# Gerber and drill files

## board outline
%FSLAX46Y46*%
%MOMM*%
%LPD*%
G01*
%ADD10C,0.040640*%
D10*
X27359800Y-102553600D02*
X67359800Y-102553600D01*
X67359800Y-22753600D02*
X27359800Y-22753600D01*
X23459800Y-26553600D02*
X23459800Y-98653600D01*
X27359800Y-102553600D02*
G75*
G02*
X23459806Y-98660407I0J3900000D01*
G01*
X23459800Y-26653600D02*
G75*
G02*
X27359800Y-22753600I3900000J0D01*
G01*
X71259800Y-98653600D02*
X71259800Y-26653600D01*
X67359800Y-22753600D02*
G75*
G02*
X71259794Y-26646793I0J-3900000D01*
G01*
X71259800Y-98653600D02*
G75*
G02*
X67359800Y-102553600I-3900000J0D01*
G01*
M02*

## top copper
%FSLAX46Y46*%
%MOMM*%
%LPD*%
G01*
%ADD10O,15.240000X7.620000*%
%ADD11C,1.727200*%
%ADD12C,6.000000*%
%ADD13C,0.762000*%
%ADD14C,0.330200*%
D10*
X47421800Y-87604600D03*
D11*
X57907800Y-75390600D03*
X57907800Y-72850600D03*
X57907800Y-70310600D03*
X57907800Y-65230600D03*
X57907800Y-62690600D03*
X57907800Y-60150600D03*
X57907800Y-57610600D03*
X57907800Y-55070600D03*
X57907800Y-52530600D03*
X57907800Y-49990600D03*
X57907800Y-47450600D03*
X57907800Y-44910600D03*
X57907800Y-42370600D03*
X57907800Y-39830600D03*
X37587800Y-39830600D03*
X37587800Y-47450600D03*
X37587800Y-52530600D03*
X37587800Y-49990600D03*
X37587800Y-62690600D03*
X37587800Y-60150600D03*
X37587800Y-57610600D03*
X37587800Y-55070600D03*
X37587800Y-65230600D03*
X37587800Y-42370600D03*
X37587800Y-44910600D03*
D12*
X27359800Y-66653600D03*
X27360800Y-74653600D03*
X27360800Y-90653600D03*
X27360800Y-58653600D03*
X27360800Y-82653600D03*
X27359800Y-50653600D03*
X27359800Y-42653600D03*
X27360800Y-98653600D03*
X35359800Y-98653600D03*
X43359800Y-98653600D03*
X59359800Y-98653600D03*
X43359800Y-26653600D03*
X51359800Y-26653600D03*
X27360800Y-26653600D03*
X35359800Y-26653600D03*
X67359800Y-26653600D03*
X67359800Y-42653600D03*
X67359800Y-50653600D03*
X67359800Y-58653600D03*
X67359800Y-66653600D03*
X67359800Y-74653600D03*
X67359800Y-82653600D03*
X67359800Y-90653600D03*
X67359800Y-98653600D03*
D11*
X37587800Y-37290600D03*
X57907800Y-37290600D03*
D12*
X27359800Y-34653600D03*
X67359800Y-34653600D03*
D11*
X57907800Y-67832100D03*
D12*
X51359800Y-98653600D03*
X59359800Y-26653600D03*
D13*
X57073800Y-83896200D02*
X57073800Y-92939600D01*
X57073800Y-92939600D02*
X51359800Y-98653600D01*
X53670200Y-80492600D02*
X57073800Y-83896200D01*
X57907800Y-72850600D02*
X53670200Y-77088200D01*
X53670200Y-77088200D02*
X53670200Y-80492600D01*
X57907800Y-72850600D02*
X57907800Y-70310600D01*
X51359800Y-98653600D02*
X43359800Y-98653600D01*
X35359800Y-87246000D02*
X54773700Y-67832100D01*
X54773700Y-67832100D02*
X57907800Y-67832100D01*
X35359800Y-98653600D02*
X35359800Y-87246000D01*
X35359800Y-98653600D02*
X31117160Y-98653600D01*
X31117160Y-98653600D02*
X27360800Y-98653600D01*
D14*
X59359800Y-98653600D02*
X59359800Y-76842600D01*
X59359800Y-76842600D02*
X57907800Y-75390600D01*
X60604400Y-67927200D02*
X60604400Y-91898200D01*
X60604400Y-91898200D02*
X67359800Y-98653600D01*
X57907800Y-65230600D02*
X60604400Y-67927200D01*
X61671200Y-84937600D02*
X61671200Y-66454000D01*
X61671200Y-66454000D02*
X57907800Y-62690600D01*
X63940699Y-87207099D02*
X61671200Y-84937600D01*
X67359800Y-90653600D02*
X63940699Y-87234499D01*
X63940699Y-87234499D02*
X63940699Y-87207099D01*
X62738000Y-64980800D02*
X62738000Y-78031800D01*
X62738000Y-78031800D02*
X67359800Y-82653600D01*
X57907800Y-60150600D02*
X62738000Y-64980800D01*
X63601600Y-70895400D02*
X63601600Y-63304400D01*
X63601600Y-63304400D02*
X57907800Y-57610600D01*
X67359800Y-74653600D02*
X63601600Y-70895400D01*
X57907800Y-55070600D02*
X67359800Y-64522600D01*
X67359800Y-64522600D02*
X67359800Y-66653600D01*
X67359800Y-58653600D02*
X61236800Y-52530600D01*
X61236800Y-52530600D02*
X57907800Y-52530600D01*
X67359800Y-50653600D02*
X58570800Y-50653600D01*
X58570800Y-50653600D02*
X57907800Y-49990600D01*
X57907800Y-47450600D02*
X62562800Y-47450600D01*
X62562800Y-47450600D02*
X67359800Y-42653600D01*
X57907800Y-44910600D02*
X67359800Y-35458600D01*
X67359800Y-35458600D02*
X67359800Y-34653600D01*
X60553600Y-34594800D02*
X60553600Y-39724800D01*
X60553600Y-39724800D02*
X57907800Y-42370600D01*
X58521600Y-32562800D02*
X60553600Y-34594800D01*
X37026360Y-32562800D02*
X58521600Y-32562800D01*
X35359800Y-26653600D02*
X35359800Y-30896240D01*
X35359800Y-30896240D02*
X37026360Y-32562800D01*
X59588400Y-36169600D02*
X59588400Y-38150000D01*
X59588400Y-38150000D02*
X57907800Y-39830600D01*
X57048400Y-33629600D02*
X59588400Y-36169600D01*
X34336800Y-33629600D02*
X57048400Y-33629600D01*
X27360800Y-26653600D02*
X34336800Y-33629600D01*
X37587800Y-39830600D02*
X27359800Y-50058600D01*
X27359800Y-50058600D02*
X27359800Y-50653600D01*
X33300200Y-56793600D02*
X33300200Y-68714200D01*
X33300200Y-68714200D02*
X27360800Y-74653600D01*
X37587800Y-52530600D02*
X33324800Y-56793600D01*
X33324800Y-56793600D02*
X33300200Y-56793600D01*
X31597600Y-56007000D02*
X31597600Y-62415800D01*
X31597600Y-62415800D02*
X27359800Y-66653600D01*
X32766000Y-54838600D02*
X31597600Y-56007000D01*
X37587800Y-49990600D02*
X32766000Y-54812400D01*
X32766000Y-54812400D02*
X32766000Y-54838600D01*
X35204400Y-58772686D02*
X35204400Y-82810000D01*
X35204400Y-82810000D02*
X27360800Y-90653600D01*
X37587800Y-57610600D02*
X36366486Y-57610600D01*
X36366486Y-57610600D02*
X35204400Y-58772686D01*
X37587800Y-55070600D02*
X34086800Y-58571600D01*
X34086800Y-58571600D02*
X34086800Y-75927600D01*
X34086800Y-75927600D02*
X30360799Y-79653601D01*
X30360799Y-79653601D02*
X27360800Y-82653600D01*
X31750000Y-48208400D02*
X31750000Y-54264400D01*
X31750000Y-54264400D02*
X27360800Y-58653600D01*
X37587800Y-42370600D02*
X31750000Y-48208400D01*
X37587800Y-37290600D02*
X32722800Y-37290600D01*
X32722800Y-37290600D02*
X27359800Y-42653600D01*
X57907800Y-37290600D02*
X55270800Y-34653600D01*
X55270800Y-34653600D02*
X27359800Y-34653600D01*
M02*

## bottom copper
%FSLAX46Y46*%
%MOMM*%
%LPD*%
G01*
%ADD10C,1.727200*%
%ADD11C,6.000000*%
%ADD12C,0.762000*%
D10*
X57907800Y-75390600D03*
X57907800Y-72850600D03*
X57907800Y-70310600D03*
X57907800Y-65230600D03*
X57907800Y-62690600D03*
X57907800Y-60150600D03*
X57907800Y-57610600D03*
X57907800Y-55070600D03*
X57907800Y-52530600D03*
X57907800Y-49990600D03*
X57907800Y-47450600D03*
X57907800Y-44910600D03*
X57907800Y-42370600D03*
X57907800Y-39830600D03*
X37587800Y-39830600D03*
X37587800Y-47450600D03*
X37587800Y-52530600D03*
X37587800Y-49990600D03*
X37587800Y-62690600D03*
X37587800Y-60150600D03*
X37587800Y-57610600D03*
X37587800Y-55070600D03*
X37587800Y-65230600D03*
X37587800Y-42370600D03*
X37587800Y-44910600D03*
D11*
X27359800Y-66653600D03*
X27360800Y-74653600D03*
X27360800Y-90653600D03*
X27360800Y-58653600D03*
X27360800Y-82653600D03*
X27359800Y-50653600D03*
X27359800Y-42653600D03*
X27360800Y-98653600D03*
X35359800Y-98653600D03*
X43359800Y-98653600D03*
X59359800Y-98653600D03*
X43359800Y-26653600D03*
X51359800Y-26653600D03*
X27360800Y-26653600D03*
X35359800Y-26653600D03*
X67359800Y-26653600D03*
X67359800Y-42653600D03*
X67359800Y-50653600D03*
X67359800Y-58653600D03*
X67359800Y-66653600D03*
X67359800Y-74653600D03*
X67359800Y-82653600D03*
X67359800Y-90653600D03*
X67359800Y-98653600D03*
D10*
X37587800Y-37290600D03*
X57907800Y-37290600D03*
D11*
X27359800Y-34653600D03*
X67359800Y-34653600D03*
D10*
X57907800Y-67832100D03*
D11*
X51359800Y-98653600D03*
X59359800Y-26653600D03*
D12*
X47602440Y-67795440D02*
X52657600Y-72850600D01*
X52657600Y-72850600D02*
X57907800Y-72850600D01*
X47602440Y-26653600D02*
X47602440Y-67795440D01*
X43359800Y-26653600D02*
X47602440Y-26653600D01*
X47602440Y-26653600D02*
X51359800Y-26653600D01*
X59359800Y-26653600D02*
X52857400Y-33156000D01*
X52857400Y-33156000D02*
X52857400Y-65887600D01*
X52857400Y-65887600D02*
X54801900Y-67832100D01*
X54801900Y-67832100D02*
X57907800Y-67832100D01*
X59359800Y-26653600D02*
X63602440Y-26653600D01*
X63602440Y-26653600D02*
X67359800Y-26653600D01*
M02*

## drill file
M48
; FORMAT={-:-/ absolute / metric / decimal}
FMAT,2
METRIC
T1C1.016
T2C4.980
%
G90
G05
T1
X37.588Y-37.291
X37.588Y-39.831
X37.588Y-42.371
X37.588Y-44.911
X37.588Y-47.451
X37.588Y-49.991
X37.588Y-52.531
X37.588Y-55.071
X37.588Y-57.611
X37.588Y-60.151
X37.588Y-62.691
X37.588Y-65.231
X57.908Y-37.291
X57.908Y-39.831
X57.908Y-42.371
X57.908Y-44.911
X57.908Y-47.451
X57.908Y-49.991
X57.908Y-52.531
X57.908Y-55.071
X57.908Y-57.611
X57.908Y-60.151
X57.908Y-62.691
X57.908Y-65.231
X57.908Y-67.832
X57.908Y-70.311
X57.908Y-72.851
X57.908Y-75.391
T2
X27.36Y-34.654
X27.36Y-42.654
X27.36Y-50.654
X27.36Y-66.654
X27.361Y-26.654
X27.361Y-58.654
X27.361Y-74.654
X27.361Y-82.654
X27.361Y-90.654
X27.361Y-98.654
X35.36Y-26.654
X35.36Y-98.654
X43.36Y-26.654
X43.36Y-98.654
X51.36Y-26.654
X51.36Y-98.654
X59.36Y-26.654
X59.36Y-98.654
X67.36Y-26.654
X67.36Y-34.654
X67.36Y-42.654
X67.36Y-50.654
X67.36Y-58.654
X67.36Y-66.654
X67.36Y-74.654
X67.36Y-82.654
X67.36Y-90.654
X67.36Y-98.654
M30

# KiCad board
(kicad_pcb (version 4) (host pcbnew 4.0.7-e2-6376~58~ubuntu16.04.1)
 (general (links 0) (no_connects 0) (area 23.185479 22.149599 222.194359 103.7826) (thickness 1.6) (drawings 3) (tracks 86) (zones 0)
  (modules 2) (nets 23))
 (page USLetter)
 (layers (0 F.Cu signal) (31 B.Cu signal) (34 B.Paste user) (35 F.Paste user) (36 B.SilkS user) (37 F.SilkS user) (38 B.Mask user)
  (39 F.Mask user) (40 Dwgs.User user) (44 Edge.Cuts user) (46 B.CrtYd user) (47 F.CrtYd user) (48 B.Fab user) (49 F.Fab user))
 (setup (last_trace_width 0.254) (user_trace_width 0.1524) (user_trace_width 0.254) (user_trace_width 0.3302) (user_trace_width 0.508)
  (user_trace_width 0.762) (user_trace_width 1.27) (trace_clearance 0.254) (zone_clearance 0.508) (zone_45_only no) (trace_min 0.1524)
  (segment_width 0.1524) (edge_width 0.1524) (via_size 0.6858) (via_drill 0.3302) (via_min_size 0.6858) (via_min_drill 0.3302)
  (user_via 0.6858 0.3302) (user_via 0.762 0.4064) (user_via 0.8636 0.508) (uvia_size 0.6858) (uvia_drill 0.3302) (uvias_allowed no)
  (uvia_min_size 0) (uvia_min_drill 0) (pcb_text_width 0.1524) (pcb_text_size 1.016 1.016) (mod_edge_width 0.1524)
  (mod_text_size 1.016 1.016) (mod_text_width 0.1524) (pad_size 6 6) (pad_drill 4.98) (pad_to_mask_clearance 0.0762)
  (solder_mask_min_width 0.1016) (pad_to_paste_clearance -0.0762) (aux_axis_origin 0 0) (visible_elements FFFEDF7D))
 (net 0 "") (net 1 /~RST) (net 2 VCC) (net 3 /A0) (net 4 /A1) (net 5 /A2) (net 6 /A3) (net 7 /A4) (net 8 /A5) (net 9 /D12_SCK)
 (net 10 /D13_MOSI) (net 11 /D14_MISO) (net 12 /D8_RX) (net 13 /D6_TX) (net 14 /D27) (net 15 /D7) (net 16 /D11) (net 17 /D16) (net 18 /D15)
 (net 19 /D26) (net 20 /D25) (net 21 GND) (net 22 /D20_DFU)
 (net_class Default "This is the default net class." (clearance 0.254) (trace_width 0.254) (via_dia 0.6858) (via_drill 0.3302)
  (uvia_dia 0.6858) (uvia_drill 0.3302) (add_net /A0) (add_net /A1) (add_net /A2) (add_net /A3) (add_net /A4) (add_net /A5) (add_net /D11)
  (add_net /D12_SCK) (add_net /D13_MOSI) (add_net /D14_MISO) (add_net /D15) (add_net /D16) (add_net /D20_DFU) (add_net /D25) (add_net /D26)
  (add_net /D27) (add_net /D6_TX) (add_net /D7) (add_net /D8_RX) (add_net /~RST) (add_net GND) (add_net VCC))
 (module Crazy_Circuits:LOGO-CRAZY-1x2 (layer F.Cu) (at 47.4218 91.5416)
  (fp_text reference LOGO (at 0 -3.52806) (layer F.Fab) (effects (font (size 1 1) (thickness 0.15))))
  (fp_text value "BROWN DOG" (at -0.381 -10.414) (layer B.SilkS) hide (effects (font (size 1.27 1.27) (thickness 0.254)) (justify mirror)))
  (pad BG smd oval (at 0 -3.937) (size 15.24 7.62) (layers F.Cu)))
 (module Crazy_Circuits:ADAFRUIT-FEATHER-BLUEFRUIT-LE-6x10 (layer F.Cu) (at 27.3598 58.6536)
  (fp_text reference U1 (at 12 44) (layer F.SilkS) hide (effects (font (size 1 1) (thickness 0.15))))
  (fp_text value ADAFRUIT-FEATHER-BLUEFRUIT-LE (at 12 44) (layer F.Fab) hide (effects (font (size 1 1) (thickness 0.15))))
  (fp_line (start 0 43.9) (end 40 43.9) (layer Edge.Cuts) (width 0.04064))
  (fp_line (start 40 -35.9) (end 0 -35.9) (layer Edge.Cuts) (width 0.04064))
  (fp_line (start -3.9 -32.1) (end -3.9 40) (layer Edge.Cuts) (width 0.04064))
  (fp_arc (start 0 40) (end 0 43.9) (angle 89.9) (layer Edge.Cuts) (width 0.04064))
  (fp_arc (start 0 -32) (end -3.9 -32) (angle 90) (layer Edge.Cuts) (width 0.04064))
  (fp_line (start 43.9 40) (end 43.9 -32) (layer Edge.Cuts) (width 0.04064))
  (fp_arc (start 40 -32) (end 40 -35.9) (angle 89.9) (layer Edge.Cuts) (width 0.04064))
  (fp_arc (start 40 40) (end 43.9 40) (angle 90) (layer Edge.Cuts) (width 0.04064))
  (pad 35 thru_hole circle (at 30.548 16.737 180) (size 1.7272 1.7272) (drill 1.016) (layers *.Cu *.Mask F.SilkS) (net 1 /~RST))
  (pad 3V thru_hole circle (at 30.548 14.197 180) (size 1.7272 1.7272) (drill 1.016) (layers *.Cu *.Mask F.SilkS) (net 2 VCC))
  (pad 3V thru_hole circle (at 30.548 11.657 180) (size 1.7272 1.7272) (drill 1.016) (layers *.Cu *.Mask F.SilkS) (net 2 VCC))
  (pad 15 thru_hole circle (at 30.548 6.577 180) (size 1.7272 1.7272) (drill 1.016) (layers *.Cu *.Mask F.SilkS) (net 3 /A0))
  (pad 16 thru_hole circle (at 30.548 4.037 180) (size 1.7272 1.7272) (drill 1.016) (layers *.Cu *.Mask F.SilkS) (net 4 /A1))
  (pad 17 thru_hole circle (at 30.548 1.497 180) (size 1.7272 1.7272) (drill 1.016) (layers *.Cu *.Mask F.SilkS) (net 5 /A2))
  (pad 18 thru_hole circle (at 30.548 -1.043 180) (size 1.7272 1.7272) (drill 1.016) (layers *.Cu *.Mask F.SilkS) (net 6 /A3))
  (pad 5 thru_hole circle (at 30.548 -3.583 180) (size 1.7272 1.7272) (drill 1.016) (layers *.Cu *.Mask F.SilkS) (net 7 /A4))
  (pad 6 thru_hole circle (at 30.548 -6.123 180) (size 1.7272 1.7272) (drill 1.016) (layers *.Cu *.Mask F.SilkS) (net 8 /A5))
  (pad 26 thru_hole circle (at 30.548 -8.663 180) (size 1.7272 1.7272) (drill 1.016) (layers *.Cu *.Mask F.SilkS) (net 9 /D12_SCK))
  (pad 27 thru_hole circle (at 30.548 -11.203 180) (size 1.7272 1.7272) (drill 1.016) (layers *.Cu *.Mask F.SilkS) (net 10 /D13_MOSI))
  (pad 28 thru_hole circle (at 30.548 -13.743 180) (size 1.7272 1.7272) (drill 1.016) (layers *.Cu *.Mask F.SilkS) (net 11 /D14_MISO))
  (pad 21 thru_hole circle (at 30.548 -16.283 180) (size 1.7272 1.7272) (drill 1.016) (layers *.Cu *.Mask F.SilkS) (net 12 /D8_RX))
  (pad 19 thru_hole circle (at 30.548 -18.823 180) (size 1.7272 1.7272) (drill 1.016) (layers *.Cu *.Mask F.SilkS) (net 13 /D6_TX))
  (pad 3 thru_hole circle (at 10.228 -18.823 180) (size 1.7272 1.7272) (drill 1.016) (layers *.Cu *.Mask F.SilkS) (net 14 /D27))
  (pad 31 thru_hole circle (at 10.228 -11.203 180) (size 1.7272 1.7272) (drill 1.016) (layers *.Cu *.Mask F.SilkS))
  (pad 20 thru_hole circle (at 10.228 -6.123 180) (size 1.7272 1.7272) (drill 1.016) (layers *.Cu *.Mask F.SilkS) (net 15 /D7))
  (pad 25 thru_hole circle (at 10.228 -8.663 180) (size 1.7272 1.7272) (drill 1.016) (layers *.Cu *.Mask F.SilkS) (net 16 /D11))
  (pad EN thru_hole circle (at 10.228 4.037 180) (size 1.7272 1.7272) (drill 1.016) (layers *.Cu *.Mask F.SilkS))
  (pad USB thru_hole circle (at 10.228 1.497 180) (size 1.7272 1.7272) (drill 1.016) (layers *.Cu *.Mask F.SilkS))
  (pad 30 thru_hole circle (at 10.228 -1.043 180) (size 1.7272 1.7272) (drill 1.016) (layers *.Cu *.Mask F.SilkS) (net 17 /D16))
  (pad 29 thru_hole circle (at 10.228 -3.583 180) (size 1.7272 1.7272) (drill 1.016) (layers *.Cu *.Mask F.SilkS) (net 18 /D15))
  (pad VBAT thru_hole circle (at 10.228 6.577 180) (size 1.7272 1.7272) (drill 1.016) (layers *.Cu *.Mask F.SilkS))
  (pad 4 thru_hole circle (at 10.228 -16.283 180) (size 1.7272 1.7272) (drill 1.016) (layers *.Cu *.Mask F.SilkS) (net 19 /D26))
  (pad 7 thru_hole circle (at 10.228 -13.743 180) (size 1.7272 1.7272) (drill 1.016) (layers *.Cu *.Mask F.SilkS))
  (pad 25 thru_hole circle (at 0 8 90) (size 6 6) (drill 4.98) (layers *.Cu *.Mask) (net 16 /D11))
  (pad 20 thru_hole circle (at 0.001 16 90) (size 6 6) (drill 4.98) (layers *.Cu *.Mask) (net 15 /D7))
  (pad 30 thru_hole circle (at 0.001 32 90) (size 6 6) (drill 4.98) (layers *.Cu *.Mask) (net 17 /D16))
  (pad 4 thru_hole circle (at 0.001 0 90) (size 6 6) (drill 4.98) (layers *.Cu *.Mask) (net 19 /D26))
  (pad 29 thru_hole circle (at 0.001 24 90) (size 6 6) (drill 4.98) (layers *.Cu *.Mask) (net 18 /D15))
  (pad 3 thru_hole circle (at 0 -8 90) (size 6 6) (drill 4.98) (layers *.Cu *.Mask) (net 14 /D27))
  (pad 2 thru_hole circle (at 0 -16 90) (size 6 6) (drill 4.98) (layers *.Cu *.Mask) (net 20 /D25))
  (pad GND thru_hole circle (at 0.001 40 90) (size 6 6) (drill 4.98) (layers *.Cu *.Mask) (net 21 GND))
  (pad GND thru_hole circle (at 8 40 90) (size 6 6) (drill 4.98) (layers *.Cu *.Mask) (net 21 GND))
  (pad 3V thru_hole circle (at 16 40 90) (size 6 6) (drill 4.98) (layers *.Cu *.Mask) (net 2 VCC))
  (pad 35 thru_hole circle (at 32 40 90) (size 6 6) (drill 4.98) (layers *.Cu *.Mask) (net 1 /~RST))
  (pad 3V thru_hole circle (at 16 -32 90) (size 6 6) (drill 4.98) (layers *.Cu *.Mask) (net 2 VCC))
  (pad 3V thru_hole circle (at 24 -32 90) (size 6 6) (drill 4.98) (layers *.Cu *.Mask) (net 2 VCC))
  (pad 19 thru_hole circle (at 0.001 -32 90) (size 6 6) (drill 4.98) (layers *.Cu *.Mask) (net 13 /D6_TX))
  (pad 21 thru_hole circle (at 8 -32 90) (size 6 6) (drill 4.98) (layers *.Cu *.Mask) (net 12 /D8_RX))
  (pad GND thru_hole circle (at 40 -32 90) (size 6 6) (drill 4.98) (layers *.Cu *.Mask) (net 21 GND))
  (pad 27 thru_hole circle (at 40 -16 90) (size 6 6) (drill 4.98) (layers *.Cu *.Mask) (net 10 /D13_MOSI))
  (pad 26 thru_hole circle (at 40 -8 90) (size 6 6) (drill 4.98) (layers *.Cu *.Mask) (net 9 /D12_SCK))
  (pad 6 thru_hole circle (at 40 0 90) (size 6 6) (drill 4.98) (layers *.Cu *.Mask) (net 8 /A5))
  (pad 5 thru_hole circle (at 40 8 90) (size 6 6) (drill 4.98) (layers *.Cu *.Mask) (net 7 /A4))
  (pad 18 thru_hole circle (at 40 16 90) (size 6 6) (drill 4.98) (layers *.Cu *.Mask) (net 6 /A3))
  (pad 17 thru_hole circle (at 40 24 90) (size 6 6) (drill 4.98) (layers *.Cu *.Mask) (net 5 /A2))
  (pad 16 thru_hole circle (at 40 32 90) (size 6 6) (drill 4.98) (layers *.Cu *.Mask) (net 4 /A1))
  (pad 15 thru_hole circle (at 40 40 90) (size 6 6) (drill 4.98) (layers *.Cu *.Mask) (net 3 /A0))
  (pad 2 thru_hole circle (at 10.228 -21.363 180) (size 1.7272 1.7272) (drill 1.016) (layers *.Cu *.Mask F.SilkS) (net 20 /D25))
  (pad 34 thru_hole circle (at 30.548 -21.363 180) (size 1.7272 1.7272) (drill 1.016) (layers *.Cu *.Mask F.SilkS) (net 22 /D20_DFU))
  (pad 34 thru_hole circle (at 0 -24 90) (size 6 6) (drill 4.98) (layers *.Cu *.Mask) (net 22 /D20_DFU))
  (pad 28 thru_hole circle (at 40 -24 90) (size 6 6) (drill 4.98) (layers *.Cu *.Mask) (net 11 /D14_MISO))
  (pad GND thru_hole circle (at 30.548 9.1785 180) (size 1.7272 1.7272) (drill 1.016) (layers *.Cu *.Mask F.SilkS) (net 21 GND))
  (pad 3V thru_hole circle (at 24 40 90) (size 6 6) (drill 4.98) (layers *.Cu *.Mask) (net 2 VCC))
  (pad GND thru_hole circle (at 32 -32 90) (size 6 6) (drill 4.98) (layers *.Cu *.Mask) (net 21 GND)))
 (segment (start 47.60244 67.79544) (end 52.6576 72.8506) (width 0.762) (layer B.Cu) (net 2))
 (segment (start 52.6576 72.8506) (end 57.9078 72.8506) (width 0.762) (layer B.Cu) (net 2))
 (segment (start 47.60244 26.6536) (end 47.60244 67.79544) (width 0.762) (layer B.Cu) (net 2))
 (segment (start 57.0738 83.8962) (end 57.0738 92.9396) (width 0.762) (layer F.Cu) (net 2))
 (segment (start 57.0738 92.9396) (end 51.3598 98.6536) (width 0.762) (layer F.Cu) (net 2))
 (segment (start 53.6702 80.4926) (end 57.0738 83.8962) (width 0.762) (layer F.Cu) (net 2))
 (segment (start 57.9078 72.8506) (end 53.6702 77.0882) (width 0.762) (layer F.Cu) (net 2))
 (segment (start 53.6702 77.0882) (end 53.6702 80.4926) (width 0.762) (layer F.Cu) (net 2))
 (segment (start 57.9078 72.8506) (end 57.9078 70.3106) (width 0.762) (layer F.Cu) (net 2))
 (segment (start 51.3598 98.6536) (end 43.3598 98.6536) (width 0.762) (layer F.Cu) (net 2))
 (segment (start 43.3598 26.6536) (end 47.60244 26.6536) (width 0.762) (layer B.Cu) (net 2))
 (segment (start 47.60244 26.6536) (end 51.3598 26.6536) (width 0.762) (layer B.Cu) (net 2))
 (segment (start 59.3598 26.6536) (end 52.8574 33.156) (width 0.762) (layer B.Cu) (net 21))
 (segment (start 52.8574 33.156) (end 52.8574 65.8876) (width 0.762) (layer B.Cu) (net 21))
 (segment (start 52.8574 65.8876) (end 54.8019 67.8321) (width 0.762) (layer B.Cu) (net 21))
 (segment (start 54.8019 67.8321) (end 57.9078 67.8321) (width 0.762) (layer B.Cu) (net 21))
 (segment (start 35.3598 87.246) (end 54.7737 67.8321) (width 0.762) (layer F.Cu) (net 21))
 (segment (start 54.7737 67.8321) (end 57.9078 67.8321) (width 0.762) (layer F.Cu) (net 21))
 (segment (start 35.3598 98.6536) (end 35.3598 87.246) (width 0.762) (layer F.Cu) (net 21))
 (segment (start 35.3598 98.6536) (end 31.11716 98.6536) (width 0.762) (layer F.Cu) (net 21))
 (segment (start 31.11716 98.6536) (end 27.3608 98.6536) (width 0.762) (layer F.Cu) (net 21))
 (segment (start 59.3598 26.6536) (end 63.60244 26.6536) (width 0.762) (layer B.Cu) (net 21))
 (segment (start 63.60244 26.6536) (end 67.3598 26.6536) (width 0.762) (layer B.Cu) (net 21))
 (segment (start 59.3598 98.6536) (end 59.3598 76.8426) (width 0.3302) (layer F.Cu) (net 1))
 (segment (start 59.3598 76.8426) (end 57.9078 75.3906) (width 0.3302) (layer F.Cu) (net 1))
 (segment (start 60.6044 67.9272) (end 60.6044 91.8982) (width 0.3302) (layer F.Cu) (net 3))
 (segment (start 60.6044 91.8982) (end 67.3598 98.6536) (width 0.3302) (layer F.Cu) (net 3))
 (segment (start 57.9078 65.2306) (end 60.6044 67.9272) (width 0.3302) (layer F.Cu) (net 3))
 (segment (start 61.6712 84.9376) (end 61.6712 66.454) (width 0.3302) (layer F.Cu) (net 4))
 (segment (start 61.6712 66.454) (end 57.9078 62.6906) (width 0.3302) (layer F.Cu) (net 4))
 (segment (start 63.940699 87.207099) (end 61.6712 84.9376) (width 0.3302) (layer F.Cu) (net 4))
 (segment (start 67.3598 90.6536) (end 63.940699 87.234499) (width 0.3302) (layer F.Cu) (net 4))
 (segment (start 63.940699 87.234499) (end 63.940699 87.207099) (width 0.3302) (layer F.Cu) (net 4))
 (segment (start 62.738 64.9808) (end 62.738 78.0318) (width 0.3302) (layer F.Cu) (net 5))
 (segment (start 62.738 78.0318) (end 67.3598 82.6536) (width 0.3302) (layer F.Cu) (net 5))
 (segment (start 57.9078 60.1506) (end 62.738 64.9808) (width 0.3302) (layer F.Cu) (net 5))
 (segment (start 63.6016 70.8954) (end 63.6016 63.3044) (width 0.3302) (layer F.Cu) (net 6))
 (segment (start 63.6016 63.3044) (end 57.9078 57.6106) (width 0.3302) (layer F.Cu) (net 6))
 (segment (start 67.3598 74.6536) (end 63.6016 70.8954) (width 0.3302) (layer F.Cu) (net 6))
 (segment (start 57.9078 55.0706) (end 67.3598 64.5226) (width 0.3302) (layer F.Cu) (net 7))
 (segment (start 67.3598 64.5226) (end 67.3598 66.6536) (width 0.3302) (layer F.Cu) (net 7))
 (segment (start 67.3598 58.6536) (end 61.2368 52.5306) (width 0.3302) (layer F.Cu) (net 8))
 (segment (start 61.2368 52.5306) (end 57.9078 52.5306) (width 0.3302) (layer F.Cu) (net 8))
 (segment (start 67.3598 50.6536) (end 58.5708 50.6536) (width 0.3302) (layer F.Cu) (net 9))
 (segment (start 58.5708 50.6536) (end 57.9078 49.9906) (width 0.3302) (layer F.Cu) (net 9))
 (segment (start 57.9078 47.4506) (end 62.5628 47.4506) (width 0.3302) (layer F.Cu) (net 10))
 (segment (start 62.5628 47.4506) (end 67.3598 42.6536) (width 0.3302) (layer F.Cu) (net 10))
 (segment (start 57.9078 44.9106) (end 67.3598 35.4586) (width 0.3302) (layer F.Cu) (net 11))
 (segment (start 67.3598 35.4586) (end 67.3598 34.6536) (width 0.3302) (layer F.Cu) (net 11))
 (segment (start 60.5536 34.5948) (end 60.5536 39.7248) (width 0.3302) (layer F.Cu) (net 12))
 (segment (start 60.5536 39.7248) (end 57.9078 42.3706) (width 0.3302) (layer F.Cu) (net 12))
 (segment (start 58.5216 32.5628) (end 60.5536 34.5948) (width 0.3302) (layer F.Cu) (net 12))
 (segment (start 37.02636 32.5628) (end 58.5216 32.5628) (width 0.3302) (layer F.Cu) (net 12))
 (segment (start 35.3598 26.6536) (end 35.3598 30.89624) (width 0.3302) (layer F.Cu) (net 12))
 (segment (start 35.3598 30.89624) (end 37.02636 32.5628) (width 0.3302) (layer F.Cu) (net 12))
 (segment (start 59.5884 36.1696) (end 59.5884 38.15) (width 0.3302) (layer F.Cu) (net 13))
 (segment (start 59.5884 38.15) (end 57.9078 39.8306) (width 0.3302) (layer F.Cu) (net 13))
 (segment (start 57.0484 33.6296) (end 59.5884 36.1696) (width 0.3302) (layer F.Cu) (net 13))
 (segment (start 34.3368 33.6296) (end 57.0484 33.6296) (width 0.3302) (layer F.Cu) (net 13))
 (segment (start 27.3608 26.6536) (end 34.3368 33.6296) (width 0.3302) (layer F.Cu) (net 13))
 (segment (start 37.5878 39.8306) (end 27.3598 50.0586) (width 0.3302) (layer F.Cu) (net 14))
 (segment (start 27.3598 50.0586) (end 27.3598 50.6536) (width 0.3302) (layer F.Cu) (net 14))
 (segment (start 33.3002 56.7936) (end 33.3002 68.7142) (width 0.3302) (layer F.Cu) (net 15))
 (segment (start 33.3002 68.7142) (end 27.3608 74.6536) (width 0.3302) (layer F.Cu) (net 15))
 (segment (start 37.5878 52.5306) (end 33.3248 56.7936) (width 0.3302) (layer F.Cu) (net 15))
 (segment (start 33.3248 56.7936) (end 33.3002 56.7936) (width 0.3302) (layer F.Cu) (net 15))
 (segment (start 31.5976 56.007) (end 31.5976 62.4158) (width 0.3302) (layer F.Cu) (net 16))
 (segment (start 31.5976 62.4158) (end 27.3598 66.6536) (width 0.3302) (layer F.Cu) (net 16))
 (segment (start 32.766 54.8386) (end 31.5976 56.007) (width 0.3302) (layer F.Cu) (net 16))
 (segment (start 37.5878 49.9906) (end 32.766 54.8124) (width 0.3302) (layer F.Cu) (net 16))
 (segment (start 32.766 54.8124) (end 32.766 54.8386) (width 0.3302) (layer F.Cu) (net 16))
 (segment (start 35.2044 58.772686) (end 35.2044 82.81) (width 0.3302) (layer F.Cu) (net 17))
 (segment (start 35.2044 82.81) (end 27.3608 90.6536) (width 0.3302) (layer F.Cu) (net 17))
 (segment (start 37.5878 57.6106) (end 36.366486 57.6106) (width 0.3302) (layer F.Cu) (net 17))
 (segment (start 36.366486 57.6106) (end 35.2044 58.772686) (width 0.3302) (layer F.Cu) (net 17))
 (segment (start 37.5878 55.0706) (end 34.0868 58.5716) (width 0.3302) (layer F.Cu) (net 18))
 (segment (start 34.0868 58.5716) (end 34.0868 75.9276) (width 0.3302) (layer F.Cu) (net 18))
 (segment (start 34.0868 75.9276) (end 30.360799 79.653601) (width 0.3302) (layer F.Cu) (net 18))
 (segment (start 30.360799 79.653601) (end 27.3608 82.6536) (width 0.3302) (layer F.Cu) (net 18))
 (segment (start 31.75 48.2084) (end 31.75 54.2644) (width 0.3302) (layer F.Cu) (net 19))
 (segment (start 31.75 54.2644) (end 27.3608 58.6536) (width 0.3302) (layer F.Cu) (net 19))
 (segment (start 37.5878 42.3706) (end 31.75 48.2084) (width 0.3302) (layer F.Cu) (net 19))
 (segment (start 37.5878 37.2906) (end 32.7228 37.2906) (width 0.3302) (layer F.Cu) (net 20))
 (segment (start 32.7228 37.2906) (end 27.3598 42.6536) (width 0.3302) (layer F.Cu) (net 20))
 (segment (start 57.9078 37.2906) (end 55.2708 34.6536) (width 0.3302) (layer F.Cu) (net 22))
 (segment (start 55.2708 34.6536) (end 27.3598 34.6536) (width 0.3302) (layer F.Cu) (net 22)))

